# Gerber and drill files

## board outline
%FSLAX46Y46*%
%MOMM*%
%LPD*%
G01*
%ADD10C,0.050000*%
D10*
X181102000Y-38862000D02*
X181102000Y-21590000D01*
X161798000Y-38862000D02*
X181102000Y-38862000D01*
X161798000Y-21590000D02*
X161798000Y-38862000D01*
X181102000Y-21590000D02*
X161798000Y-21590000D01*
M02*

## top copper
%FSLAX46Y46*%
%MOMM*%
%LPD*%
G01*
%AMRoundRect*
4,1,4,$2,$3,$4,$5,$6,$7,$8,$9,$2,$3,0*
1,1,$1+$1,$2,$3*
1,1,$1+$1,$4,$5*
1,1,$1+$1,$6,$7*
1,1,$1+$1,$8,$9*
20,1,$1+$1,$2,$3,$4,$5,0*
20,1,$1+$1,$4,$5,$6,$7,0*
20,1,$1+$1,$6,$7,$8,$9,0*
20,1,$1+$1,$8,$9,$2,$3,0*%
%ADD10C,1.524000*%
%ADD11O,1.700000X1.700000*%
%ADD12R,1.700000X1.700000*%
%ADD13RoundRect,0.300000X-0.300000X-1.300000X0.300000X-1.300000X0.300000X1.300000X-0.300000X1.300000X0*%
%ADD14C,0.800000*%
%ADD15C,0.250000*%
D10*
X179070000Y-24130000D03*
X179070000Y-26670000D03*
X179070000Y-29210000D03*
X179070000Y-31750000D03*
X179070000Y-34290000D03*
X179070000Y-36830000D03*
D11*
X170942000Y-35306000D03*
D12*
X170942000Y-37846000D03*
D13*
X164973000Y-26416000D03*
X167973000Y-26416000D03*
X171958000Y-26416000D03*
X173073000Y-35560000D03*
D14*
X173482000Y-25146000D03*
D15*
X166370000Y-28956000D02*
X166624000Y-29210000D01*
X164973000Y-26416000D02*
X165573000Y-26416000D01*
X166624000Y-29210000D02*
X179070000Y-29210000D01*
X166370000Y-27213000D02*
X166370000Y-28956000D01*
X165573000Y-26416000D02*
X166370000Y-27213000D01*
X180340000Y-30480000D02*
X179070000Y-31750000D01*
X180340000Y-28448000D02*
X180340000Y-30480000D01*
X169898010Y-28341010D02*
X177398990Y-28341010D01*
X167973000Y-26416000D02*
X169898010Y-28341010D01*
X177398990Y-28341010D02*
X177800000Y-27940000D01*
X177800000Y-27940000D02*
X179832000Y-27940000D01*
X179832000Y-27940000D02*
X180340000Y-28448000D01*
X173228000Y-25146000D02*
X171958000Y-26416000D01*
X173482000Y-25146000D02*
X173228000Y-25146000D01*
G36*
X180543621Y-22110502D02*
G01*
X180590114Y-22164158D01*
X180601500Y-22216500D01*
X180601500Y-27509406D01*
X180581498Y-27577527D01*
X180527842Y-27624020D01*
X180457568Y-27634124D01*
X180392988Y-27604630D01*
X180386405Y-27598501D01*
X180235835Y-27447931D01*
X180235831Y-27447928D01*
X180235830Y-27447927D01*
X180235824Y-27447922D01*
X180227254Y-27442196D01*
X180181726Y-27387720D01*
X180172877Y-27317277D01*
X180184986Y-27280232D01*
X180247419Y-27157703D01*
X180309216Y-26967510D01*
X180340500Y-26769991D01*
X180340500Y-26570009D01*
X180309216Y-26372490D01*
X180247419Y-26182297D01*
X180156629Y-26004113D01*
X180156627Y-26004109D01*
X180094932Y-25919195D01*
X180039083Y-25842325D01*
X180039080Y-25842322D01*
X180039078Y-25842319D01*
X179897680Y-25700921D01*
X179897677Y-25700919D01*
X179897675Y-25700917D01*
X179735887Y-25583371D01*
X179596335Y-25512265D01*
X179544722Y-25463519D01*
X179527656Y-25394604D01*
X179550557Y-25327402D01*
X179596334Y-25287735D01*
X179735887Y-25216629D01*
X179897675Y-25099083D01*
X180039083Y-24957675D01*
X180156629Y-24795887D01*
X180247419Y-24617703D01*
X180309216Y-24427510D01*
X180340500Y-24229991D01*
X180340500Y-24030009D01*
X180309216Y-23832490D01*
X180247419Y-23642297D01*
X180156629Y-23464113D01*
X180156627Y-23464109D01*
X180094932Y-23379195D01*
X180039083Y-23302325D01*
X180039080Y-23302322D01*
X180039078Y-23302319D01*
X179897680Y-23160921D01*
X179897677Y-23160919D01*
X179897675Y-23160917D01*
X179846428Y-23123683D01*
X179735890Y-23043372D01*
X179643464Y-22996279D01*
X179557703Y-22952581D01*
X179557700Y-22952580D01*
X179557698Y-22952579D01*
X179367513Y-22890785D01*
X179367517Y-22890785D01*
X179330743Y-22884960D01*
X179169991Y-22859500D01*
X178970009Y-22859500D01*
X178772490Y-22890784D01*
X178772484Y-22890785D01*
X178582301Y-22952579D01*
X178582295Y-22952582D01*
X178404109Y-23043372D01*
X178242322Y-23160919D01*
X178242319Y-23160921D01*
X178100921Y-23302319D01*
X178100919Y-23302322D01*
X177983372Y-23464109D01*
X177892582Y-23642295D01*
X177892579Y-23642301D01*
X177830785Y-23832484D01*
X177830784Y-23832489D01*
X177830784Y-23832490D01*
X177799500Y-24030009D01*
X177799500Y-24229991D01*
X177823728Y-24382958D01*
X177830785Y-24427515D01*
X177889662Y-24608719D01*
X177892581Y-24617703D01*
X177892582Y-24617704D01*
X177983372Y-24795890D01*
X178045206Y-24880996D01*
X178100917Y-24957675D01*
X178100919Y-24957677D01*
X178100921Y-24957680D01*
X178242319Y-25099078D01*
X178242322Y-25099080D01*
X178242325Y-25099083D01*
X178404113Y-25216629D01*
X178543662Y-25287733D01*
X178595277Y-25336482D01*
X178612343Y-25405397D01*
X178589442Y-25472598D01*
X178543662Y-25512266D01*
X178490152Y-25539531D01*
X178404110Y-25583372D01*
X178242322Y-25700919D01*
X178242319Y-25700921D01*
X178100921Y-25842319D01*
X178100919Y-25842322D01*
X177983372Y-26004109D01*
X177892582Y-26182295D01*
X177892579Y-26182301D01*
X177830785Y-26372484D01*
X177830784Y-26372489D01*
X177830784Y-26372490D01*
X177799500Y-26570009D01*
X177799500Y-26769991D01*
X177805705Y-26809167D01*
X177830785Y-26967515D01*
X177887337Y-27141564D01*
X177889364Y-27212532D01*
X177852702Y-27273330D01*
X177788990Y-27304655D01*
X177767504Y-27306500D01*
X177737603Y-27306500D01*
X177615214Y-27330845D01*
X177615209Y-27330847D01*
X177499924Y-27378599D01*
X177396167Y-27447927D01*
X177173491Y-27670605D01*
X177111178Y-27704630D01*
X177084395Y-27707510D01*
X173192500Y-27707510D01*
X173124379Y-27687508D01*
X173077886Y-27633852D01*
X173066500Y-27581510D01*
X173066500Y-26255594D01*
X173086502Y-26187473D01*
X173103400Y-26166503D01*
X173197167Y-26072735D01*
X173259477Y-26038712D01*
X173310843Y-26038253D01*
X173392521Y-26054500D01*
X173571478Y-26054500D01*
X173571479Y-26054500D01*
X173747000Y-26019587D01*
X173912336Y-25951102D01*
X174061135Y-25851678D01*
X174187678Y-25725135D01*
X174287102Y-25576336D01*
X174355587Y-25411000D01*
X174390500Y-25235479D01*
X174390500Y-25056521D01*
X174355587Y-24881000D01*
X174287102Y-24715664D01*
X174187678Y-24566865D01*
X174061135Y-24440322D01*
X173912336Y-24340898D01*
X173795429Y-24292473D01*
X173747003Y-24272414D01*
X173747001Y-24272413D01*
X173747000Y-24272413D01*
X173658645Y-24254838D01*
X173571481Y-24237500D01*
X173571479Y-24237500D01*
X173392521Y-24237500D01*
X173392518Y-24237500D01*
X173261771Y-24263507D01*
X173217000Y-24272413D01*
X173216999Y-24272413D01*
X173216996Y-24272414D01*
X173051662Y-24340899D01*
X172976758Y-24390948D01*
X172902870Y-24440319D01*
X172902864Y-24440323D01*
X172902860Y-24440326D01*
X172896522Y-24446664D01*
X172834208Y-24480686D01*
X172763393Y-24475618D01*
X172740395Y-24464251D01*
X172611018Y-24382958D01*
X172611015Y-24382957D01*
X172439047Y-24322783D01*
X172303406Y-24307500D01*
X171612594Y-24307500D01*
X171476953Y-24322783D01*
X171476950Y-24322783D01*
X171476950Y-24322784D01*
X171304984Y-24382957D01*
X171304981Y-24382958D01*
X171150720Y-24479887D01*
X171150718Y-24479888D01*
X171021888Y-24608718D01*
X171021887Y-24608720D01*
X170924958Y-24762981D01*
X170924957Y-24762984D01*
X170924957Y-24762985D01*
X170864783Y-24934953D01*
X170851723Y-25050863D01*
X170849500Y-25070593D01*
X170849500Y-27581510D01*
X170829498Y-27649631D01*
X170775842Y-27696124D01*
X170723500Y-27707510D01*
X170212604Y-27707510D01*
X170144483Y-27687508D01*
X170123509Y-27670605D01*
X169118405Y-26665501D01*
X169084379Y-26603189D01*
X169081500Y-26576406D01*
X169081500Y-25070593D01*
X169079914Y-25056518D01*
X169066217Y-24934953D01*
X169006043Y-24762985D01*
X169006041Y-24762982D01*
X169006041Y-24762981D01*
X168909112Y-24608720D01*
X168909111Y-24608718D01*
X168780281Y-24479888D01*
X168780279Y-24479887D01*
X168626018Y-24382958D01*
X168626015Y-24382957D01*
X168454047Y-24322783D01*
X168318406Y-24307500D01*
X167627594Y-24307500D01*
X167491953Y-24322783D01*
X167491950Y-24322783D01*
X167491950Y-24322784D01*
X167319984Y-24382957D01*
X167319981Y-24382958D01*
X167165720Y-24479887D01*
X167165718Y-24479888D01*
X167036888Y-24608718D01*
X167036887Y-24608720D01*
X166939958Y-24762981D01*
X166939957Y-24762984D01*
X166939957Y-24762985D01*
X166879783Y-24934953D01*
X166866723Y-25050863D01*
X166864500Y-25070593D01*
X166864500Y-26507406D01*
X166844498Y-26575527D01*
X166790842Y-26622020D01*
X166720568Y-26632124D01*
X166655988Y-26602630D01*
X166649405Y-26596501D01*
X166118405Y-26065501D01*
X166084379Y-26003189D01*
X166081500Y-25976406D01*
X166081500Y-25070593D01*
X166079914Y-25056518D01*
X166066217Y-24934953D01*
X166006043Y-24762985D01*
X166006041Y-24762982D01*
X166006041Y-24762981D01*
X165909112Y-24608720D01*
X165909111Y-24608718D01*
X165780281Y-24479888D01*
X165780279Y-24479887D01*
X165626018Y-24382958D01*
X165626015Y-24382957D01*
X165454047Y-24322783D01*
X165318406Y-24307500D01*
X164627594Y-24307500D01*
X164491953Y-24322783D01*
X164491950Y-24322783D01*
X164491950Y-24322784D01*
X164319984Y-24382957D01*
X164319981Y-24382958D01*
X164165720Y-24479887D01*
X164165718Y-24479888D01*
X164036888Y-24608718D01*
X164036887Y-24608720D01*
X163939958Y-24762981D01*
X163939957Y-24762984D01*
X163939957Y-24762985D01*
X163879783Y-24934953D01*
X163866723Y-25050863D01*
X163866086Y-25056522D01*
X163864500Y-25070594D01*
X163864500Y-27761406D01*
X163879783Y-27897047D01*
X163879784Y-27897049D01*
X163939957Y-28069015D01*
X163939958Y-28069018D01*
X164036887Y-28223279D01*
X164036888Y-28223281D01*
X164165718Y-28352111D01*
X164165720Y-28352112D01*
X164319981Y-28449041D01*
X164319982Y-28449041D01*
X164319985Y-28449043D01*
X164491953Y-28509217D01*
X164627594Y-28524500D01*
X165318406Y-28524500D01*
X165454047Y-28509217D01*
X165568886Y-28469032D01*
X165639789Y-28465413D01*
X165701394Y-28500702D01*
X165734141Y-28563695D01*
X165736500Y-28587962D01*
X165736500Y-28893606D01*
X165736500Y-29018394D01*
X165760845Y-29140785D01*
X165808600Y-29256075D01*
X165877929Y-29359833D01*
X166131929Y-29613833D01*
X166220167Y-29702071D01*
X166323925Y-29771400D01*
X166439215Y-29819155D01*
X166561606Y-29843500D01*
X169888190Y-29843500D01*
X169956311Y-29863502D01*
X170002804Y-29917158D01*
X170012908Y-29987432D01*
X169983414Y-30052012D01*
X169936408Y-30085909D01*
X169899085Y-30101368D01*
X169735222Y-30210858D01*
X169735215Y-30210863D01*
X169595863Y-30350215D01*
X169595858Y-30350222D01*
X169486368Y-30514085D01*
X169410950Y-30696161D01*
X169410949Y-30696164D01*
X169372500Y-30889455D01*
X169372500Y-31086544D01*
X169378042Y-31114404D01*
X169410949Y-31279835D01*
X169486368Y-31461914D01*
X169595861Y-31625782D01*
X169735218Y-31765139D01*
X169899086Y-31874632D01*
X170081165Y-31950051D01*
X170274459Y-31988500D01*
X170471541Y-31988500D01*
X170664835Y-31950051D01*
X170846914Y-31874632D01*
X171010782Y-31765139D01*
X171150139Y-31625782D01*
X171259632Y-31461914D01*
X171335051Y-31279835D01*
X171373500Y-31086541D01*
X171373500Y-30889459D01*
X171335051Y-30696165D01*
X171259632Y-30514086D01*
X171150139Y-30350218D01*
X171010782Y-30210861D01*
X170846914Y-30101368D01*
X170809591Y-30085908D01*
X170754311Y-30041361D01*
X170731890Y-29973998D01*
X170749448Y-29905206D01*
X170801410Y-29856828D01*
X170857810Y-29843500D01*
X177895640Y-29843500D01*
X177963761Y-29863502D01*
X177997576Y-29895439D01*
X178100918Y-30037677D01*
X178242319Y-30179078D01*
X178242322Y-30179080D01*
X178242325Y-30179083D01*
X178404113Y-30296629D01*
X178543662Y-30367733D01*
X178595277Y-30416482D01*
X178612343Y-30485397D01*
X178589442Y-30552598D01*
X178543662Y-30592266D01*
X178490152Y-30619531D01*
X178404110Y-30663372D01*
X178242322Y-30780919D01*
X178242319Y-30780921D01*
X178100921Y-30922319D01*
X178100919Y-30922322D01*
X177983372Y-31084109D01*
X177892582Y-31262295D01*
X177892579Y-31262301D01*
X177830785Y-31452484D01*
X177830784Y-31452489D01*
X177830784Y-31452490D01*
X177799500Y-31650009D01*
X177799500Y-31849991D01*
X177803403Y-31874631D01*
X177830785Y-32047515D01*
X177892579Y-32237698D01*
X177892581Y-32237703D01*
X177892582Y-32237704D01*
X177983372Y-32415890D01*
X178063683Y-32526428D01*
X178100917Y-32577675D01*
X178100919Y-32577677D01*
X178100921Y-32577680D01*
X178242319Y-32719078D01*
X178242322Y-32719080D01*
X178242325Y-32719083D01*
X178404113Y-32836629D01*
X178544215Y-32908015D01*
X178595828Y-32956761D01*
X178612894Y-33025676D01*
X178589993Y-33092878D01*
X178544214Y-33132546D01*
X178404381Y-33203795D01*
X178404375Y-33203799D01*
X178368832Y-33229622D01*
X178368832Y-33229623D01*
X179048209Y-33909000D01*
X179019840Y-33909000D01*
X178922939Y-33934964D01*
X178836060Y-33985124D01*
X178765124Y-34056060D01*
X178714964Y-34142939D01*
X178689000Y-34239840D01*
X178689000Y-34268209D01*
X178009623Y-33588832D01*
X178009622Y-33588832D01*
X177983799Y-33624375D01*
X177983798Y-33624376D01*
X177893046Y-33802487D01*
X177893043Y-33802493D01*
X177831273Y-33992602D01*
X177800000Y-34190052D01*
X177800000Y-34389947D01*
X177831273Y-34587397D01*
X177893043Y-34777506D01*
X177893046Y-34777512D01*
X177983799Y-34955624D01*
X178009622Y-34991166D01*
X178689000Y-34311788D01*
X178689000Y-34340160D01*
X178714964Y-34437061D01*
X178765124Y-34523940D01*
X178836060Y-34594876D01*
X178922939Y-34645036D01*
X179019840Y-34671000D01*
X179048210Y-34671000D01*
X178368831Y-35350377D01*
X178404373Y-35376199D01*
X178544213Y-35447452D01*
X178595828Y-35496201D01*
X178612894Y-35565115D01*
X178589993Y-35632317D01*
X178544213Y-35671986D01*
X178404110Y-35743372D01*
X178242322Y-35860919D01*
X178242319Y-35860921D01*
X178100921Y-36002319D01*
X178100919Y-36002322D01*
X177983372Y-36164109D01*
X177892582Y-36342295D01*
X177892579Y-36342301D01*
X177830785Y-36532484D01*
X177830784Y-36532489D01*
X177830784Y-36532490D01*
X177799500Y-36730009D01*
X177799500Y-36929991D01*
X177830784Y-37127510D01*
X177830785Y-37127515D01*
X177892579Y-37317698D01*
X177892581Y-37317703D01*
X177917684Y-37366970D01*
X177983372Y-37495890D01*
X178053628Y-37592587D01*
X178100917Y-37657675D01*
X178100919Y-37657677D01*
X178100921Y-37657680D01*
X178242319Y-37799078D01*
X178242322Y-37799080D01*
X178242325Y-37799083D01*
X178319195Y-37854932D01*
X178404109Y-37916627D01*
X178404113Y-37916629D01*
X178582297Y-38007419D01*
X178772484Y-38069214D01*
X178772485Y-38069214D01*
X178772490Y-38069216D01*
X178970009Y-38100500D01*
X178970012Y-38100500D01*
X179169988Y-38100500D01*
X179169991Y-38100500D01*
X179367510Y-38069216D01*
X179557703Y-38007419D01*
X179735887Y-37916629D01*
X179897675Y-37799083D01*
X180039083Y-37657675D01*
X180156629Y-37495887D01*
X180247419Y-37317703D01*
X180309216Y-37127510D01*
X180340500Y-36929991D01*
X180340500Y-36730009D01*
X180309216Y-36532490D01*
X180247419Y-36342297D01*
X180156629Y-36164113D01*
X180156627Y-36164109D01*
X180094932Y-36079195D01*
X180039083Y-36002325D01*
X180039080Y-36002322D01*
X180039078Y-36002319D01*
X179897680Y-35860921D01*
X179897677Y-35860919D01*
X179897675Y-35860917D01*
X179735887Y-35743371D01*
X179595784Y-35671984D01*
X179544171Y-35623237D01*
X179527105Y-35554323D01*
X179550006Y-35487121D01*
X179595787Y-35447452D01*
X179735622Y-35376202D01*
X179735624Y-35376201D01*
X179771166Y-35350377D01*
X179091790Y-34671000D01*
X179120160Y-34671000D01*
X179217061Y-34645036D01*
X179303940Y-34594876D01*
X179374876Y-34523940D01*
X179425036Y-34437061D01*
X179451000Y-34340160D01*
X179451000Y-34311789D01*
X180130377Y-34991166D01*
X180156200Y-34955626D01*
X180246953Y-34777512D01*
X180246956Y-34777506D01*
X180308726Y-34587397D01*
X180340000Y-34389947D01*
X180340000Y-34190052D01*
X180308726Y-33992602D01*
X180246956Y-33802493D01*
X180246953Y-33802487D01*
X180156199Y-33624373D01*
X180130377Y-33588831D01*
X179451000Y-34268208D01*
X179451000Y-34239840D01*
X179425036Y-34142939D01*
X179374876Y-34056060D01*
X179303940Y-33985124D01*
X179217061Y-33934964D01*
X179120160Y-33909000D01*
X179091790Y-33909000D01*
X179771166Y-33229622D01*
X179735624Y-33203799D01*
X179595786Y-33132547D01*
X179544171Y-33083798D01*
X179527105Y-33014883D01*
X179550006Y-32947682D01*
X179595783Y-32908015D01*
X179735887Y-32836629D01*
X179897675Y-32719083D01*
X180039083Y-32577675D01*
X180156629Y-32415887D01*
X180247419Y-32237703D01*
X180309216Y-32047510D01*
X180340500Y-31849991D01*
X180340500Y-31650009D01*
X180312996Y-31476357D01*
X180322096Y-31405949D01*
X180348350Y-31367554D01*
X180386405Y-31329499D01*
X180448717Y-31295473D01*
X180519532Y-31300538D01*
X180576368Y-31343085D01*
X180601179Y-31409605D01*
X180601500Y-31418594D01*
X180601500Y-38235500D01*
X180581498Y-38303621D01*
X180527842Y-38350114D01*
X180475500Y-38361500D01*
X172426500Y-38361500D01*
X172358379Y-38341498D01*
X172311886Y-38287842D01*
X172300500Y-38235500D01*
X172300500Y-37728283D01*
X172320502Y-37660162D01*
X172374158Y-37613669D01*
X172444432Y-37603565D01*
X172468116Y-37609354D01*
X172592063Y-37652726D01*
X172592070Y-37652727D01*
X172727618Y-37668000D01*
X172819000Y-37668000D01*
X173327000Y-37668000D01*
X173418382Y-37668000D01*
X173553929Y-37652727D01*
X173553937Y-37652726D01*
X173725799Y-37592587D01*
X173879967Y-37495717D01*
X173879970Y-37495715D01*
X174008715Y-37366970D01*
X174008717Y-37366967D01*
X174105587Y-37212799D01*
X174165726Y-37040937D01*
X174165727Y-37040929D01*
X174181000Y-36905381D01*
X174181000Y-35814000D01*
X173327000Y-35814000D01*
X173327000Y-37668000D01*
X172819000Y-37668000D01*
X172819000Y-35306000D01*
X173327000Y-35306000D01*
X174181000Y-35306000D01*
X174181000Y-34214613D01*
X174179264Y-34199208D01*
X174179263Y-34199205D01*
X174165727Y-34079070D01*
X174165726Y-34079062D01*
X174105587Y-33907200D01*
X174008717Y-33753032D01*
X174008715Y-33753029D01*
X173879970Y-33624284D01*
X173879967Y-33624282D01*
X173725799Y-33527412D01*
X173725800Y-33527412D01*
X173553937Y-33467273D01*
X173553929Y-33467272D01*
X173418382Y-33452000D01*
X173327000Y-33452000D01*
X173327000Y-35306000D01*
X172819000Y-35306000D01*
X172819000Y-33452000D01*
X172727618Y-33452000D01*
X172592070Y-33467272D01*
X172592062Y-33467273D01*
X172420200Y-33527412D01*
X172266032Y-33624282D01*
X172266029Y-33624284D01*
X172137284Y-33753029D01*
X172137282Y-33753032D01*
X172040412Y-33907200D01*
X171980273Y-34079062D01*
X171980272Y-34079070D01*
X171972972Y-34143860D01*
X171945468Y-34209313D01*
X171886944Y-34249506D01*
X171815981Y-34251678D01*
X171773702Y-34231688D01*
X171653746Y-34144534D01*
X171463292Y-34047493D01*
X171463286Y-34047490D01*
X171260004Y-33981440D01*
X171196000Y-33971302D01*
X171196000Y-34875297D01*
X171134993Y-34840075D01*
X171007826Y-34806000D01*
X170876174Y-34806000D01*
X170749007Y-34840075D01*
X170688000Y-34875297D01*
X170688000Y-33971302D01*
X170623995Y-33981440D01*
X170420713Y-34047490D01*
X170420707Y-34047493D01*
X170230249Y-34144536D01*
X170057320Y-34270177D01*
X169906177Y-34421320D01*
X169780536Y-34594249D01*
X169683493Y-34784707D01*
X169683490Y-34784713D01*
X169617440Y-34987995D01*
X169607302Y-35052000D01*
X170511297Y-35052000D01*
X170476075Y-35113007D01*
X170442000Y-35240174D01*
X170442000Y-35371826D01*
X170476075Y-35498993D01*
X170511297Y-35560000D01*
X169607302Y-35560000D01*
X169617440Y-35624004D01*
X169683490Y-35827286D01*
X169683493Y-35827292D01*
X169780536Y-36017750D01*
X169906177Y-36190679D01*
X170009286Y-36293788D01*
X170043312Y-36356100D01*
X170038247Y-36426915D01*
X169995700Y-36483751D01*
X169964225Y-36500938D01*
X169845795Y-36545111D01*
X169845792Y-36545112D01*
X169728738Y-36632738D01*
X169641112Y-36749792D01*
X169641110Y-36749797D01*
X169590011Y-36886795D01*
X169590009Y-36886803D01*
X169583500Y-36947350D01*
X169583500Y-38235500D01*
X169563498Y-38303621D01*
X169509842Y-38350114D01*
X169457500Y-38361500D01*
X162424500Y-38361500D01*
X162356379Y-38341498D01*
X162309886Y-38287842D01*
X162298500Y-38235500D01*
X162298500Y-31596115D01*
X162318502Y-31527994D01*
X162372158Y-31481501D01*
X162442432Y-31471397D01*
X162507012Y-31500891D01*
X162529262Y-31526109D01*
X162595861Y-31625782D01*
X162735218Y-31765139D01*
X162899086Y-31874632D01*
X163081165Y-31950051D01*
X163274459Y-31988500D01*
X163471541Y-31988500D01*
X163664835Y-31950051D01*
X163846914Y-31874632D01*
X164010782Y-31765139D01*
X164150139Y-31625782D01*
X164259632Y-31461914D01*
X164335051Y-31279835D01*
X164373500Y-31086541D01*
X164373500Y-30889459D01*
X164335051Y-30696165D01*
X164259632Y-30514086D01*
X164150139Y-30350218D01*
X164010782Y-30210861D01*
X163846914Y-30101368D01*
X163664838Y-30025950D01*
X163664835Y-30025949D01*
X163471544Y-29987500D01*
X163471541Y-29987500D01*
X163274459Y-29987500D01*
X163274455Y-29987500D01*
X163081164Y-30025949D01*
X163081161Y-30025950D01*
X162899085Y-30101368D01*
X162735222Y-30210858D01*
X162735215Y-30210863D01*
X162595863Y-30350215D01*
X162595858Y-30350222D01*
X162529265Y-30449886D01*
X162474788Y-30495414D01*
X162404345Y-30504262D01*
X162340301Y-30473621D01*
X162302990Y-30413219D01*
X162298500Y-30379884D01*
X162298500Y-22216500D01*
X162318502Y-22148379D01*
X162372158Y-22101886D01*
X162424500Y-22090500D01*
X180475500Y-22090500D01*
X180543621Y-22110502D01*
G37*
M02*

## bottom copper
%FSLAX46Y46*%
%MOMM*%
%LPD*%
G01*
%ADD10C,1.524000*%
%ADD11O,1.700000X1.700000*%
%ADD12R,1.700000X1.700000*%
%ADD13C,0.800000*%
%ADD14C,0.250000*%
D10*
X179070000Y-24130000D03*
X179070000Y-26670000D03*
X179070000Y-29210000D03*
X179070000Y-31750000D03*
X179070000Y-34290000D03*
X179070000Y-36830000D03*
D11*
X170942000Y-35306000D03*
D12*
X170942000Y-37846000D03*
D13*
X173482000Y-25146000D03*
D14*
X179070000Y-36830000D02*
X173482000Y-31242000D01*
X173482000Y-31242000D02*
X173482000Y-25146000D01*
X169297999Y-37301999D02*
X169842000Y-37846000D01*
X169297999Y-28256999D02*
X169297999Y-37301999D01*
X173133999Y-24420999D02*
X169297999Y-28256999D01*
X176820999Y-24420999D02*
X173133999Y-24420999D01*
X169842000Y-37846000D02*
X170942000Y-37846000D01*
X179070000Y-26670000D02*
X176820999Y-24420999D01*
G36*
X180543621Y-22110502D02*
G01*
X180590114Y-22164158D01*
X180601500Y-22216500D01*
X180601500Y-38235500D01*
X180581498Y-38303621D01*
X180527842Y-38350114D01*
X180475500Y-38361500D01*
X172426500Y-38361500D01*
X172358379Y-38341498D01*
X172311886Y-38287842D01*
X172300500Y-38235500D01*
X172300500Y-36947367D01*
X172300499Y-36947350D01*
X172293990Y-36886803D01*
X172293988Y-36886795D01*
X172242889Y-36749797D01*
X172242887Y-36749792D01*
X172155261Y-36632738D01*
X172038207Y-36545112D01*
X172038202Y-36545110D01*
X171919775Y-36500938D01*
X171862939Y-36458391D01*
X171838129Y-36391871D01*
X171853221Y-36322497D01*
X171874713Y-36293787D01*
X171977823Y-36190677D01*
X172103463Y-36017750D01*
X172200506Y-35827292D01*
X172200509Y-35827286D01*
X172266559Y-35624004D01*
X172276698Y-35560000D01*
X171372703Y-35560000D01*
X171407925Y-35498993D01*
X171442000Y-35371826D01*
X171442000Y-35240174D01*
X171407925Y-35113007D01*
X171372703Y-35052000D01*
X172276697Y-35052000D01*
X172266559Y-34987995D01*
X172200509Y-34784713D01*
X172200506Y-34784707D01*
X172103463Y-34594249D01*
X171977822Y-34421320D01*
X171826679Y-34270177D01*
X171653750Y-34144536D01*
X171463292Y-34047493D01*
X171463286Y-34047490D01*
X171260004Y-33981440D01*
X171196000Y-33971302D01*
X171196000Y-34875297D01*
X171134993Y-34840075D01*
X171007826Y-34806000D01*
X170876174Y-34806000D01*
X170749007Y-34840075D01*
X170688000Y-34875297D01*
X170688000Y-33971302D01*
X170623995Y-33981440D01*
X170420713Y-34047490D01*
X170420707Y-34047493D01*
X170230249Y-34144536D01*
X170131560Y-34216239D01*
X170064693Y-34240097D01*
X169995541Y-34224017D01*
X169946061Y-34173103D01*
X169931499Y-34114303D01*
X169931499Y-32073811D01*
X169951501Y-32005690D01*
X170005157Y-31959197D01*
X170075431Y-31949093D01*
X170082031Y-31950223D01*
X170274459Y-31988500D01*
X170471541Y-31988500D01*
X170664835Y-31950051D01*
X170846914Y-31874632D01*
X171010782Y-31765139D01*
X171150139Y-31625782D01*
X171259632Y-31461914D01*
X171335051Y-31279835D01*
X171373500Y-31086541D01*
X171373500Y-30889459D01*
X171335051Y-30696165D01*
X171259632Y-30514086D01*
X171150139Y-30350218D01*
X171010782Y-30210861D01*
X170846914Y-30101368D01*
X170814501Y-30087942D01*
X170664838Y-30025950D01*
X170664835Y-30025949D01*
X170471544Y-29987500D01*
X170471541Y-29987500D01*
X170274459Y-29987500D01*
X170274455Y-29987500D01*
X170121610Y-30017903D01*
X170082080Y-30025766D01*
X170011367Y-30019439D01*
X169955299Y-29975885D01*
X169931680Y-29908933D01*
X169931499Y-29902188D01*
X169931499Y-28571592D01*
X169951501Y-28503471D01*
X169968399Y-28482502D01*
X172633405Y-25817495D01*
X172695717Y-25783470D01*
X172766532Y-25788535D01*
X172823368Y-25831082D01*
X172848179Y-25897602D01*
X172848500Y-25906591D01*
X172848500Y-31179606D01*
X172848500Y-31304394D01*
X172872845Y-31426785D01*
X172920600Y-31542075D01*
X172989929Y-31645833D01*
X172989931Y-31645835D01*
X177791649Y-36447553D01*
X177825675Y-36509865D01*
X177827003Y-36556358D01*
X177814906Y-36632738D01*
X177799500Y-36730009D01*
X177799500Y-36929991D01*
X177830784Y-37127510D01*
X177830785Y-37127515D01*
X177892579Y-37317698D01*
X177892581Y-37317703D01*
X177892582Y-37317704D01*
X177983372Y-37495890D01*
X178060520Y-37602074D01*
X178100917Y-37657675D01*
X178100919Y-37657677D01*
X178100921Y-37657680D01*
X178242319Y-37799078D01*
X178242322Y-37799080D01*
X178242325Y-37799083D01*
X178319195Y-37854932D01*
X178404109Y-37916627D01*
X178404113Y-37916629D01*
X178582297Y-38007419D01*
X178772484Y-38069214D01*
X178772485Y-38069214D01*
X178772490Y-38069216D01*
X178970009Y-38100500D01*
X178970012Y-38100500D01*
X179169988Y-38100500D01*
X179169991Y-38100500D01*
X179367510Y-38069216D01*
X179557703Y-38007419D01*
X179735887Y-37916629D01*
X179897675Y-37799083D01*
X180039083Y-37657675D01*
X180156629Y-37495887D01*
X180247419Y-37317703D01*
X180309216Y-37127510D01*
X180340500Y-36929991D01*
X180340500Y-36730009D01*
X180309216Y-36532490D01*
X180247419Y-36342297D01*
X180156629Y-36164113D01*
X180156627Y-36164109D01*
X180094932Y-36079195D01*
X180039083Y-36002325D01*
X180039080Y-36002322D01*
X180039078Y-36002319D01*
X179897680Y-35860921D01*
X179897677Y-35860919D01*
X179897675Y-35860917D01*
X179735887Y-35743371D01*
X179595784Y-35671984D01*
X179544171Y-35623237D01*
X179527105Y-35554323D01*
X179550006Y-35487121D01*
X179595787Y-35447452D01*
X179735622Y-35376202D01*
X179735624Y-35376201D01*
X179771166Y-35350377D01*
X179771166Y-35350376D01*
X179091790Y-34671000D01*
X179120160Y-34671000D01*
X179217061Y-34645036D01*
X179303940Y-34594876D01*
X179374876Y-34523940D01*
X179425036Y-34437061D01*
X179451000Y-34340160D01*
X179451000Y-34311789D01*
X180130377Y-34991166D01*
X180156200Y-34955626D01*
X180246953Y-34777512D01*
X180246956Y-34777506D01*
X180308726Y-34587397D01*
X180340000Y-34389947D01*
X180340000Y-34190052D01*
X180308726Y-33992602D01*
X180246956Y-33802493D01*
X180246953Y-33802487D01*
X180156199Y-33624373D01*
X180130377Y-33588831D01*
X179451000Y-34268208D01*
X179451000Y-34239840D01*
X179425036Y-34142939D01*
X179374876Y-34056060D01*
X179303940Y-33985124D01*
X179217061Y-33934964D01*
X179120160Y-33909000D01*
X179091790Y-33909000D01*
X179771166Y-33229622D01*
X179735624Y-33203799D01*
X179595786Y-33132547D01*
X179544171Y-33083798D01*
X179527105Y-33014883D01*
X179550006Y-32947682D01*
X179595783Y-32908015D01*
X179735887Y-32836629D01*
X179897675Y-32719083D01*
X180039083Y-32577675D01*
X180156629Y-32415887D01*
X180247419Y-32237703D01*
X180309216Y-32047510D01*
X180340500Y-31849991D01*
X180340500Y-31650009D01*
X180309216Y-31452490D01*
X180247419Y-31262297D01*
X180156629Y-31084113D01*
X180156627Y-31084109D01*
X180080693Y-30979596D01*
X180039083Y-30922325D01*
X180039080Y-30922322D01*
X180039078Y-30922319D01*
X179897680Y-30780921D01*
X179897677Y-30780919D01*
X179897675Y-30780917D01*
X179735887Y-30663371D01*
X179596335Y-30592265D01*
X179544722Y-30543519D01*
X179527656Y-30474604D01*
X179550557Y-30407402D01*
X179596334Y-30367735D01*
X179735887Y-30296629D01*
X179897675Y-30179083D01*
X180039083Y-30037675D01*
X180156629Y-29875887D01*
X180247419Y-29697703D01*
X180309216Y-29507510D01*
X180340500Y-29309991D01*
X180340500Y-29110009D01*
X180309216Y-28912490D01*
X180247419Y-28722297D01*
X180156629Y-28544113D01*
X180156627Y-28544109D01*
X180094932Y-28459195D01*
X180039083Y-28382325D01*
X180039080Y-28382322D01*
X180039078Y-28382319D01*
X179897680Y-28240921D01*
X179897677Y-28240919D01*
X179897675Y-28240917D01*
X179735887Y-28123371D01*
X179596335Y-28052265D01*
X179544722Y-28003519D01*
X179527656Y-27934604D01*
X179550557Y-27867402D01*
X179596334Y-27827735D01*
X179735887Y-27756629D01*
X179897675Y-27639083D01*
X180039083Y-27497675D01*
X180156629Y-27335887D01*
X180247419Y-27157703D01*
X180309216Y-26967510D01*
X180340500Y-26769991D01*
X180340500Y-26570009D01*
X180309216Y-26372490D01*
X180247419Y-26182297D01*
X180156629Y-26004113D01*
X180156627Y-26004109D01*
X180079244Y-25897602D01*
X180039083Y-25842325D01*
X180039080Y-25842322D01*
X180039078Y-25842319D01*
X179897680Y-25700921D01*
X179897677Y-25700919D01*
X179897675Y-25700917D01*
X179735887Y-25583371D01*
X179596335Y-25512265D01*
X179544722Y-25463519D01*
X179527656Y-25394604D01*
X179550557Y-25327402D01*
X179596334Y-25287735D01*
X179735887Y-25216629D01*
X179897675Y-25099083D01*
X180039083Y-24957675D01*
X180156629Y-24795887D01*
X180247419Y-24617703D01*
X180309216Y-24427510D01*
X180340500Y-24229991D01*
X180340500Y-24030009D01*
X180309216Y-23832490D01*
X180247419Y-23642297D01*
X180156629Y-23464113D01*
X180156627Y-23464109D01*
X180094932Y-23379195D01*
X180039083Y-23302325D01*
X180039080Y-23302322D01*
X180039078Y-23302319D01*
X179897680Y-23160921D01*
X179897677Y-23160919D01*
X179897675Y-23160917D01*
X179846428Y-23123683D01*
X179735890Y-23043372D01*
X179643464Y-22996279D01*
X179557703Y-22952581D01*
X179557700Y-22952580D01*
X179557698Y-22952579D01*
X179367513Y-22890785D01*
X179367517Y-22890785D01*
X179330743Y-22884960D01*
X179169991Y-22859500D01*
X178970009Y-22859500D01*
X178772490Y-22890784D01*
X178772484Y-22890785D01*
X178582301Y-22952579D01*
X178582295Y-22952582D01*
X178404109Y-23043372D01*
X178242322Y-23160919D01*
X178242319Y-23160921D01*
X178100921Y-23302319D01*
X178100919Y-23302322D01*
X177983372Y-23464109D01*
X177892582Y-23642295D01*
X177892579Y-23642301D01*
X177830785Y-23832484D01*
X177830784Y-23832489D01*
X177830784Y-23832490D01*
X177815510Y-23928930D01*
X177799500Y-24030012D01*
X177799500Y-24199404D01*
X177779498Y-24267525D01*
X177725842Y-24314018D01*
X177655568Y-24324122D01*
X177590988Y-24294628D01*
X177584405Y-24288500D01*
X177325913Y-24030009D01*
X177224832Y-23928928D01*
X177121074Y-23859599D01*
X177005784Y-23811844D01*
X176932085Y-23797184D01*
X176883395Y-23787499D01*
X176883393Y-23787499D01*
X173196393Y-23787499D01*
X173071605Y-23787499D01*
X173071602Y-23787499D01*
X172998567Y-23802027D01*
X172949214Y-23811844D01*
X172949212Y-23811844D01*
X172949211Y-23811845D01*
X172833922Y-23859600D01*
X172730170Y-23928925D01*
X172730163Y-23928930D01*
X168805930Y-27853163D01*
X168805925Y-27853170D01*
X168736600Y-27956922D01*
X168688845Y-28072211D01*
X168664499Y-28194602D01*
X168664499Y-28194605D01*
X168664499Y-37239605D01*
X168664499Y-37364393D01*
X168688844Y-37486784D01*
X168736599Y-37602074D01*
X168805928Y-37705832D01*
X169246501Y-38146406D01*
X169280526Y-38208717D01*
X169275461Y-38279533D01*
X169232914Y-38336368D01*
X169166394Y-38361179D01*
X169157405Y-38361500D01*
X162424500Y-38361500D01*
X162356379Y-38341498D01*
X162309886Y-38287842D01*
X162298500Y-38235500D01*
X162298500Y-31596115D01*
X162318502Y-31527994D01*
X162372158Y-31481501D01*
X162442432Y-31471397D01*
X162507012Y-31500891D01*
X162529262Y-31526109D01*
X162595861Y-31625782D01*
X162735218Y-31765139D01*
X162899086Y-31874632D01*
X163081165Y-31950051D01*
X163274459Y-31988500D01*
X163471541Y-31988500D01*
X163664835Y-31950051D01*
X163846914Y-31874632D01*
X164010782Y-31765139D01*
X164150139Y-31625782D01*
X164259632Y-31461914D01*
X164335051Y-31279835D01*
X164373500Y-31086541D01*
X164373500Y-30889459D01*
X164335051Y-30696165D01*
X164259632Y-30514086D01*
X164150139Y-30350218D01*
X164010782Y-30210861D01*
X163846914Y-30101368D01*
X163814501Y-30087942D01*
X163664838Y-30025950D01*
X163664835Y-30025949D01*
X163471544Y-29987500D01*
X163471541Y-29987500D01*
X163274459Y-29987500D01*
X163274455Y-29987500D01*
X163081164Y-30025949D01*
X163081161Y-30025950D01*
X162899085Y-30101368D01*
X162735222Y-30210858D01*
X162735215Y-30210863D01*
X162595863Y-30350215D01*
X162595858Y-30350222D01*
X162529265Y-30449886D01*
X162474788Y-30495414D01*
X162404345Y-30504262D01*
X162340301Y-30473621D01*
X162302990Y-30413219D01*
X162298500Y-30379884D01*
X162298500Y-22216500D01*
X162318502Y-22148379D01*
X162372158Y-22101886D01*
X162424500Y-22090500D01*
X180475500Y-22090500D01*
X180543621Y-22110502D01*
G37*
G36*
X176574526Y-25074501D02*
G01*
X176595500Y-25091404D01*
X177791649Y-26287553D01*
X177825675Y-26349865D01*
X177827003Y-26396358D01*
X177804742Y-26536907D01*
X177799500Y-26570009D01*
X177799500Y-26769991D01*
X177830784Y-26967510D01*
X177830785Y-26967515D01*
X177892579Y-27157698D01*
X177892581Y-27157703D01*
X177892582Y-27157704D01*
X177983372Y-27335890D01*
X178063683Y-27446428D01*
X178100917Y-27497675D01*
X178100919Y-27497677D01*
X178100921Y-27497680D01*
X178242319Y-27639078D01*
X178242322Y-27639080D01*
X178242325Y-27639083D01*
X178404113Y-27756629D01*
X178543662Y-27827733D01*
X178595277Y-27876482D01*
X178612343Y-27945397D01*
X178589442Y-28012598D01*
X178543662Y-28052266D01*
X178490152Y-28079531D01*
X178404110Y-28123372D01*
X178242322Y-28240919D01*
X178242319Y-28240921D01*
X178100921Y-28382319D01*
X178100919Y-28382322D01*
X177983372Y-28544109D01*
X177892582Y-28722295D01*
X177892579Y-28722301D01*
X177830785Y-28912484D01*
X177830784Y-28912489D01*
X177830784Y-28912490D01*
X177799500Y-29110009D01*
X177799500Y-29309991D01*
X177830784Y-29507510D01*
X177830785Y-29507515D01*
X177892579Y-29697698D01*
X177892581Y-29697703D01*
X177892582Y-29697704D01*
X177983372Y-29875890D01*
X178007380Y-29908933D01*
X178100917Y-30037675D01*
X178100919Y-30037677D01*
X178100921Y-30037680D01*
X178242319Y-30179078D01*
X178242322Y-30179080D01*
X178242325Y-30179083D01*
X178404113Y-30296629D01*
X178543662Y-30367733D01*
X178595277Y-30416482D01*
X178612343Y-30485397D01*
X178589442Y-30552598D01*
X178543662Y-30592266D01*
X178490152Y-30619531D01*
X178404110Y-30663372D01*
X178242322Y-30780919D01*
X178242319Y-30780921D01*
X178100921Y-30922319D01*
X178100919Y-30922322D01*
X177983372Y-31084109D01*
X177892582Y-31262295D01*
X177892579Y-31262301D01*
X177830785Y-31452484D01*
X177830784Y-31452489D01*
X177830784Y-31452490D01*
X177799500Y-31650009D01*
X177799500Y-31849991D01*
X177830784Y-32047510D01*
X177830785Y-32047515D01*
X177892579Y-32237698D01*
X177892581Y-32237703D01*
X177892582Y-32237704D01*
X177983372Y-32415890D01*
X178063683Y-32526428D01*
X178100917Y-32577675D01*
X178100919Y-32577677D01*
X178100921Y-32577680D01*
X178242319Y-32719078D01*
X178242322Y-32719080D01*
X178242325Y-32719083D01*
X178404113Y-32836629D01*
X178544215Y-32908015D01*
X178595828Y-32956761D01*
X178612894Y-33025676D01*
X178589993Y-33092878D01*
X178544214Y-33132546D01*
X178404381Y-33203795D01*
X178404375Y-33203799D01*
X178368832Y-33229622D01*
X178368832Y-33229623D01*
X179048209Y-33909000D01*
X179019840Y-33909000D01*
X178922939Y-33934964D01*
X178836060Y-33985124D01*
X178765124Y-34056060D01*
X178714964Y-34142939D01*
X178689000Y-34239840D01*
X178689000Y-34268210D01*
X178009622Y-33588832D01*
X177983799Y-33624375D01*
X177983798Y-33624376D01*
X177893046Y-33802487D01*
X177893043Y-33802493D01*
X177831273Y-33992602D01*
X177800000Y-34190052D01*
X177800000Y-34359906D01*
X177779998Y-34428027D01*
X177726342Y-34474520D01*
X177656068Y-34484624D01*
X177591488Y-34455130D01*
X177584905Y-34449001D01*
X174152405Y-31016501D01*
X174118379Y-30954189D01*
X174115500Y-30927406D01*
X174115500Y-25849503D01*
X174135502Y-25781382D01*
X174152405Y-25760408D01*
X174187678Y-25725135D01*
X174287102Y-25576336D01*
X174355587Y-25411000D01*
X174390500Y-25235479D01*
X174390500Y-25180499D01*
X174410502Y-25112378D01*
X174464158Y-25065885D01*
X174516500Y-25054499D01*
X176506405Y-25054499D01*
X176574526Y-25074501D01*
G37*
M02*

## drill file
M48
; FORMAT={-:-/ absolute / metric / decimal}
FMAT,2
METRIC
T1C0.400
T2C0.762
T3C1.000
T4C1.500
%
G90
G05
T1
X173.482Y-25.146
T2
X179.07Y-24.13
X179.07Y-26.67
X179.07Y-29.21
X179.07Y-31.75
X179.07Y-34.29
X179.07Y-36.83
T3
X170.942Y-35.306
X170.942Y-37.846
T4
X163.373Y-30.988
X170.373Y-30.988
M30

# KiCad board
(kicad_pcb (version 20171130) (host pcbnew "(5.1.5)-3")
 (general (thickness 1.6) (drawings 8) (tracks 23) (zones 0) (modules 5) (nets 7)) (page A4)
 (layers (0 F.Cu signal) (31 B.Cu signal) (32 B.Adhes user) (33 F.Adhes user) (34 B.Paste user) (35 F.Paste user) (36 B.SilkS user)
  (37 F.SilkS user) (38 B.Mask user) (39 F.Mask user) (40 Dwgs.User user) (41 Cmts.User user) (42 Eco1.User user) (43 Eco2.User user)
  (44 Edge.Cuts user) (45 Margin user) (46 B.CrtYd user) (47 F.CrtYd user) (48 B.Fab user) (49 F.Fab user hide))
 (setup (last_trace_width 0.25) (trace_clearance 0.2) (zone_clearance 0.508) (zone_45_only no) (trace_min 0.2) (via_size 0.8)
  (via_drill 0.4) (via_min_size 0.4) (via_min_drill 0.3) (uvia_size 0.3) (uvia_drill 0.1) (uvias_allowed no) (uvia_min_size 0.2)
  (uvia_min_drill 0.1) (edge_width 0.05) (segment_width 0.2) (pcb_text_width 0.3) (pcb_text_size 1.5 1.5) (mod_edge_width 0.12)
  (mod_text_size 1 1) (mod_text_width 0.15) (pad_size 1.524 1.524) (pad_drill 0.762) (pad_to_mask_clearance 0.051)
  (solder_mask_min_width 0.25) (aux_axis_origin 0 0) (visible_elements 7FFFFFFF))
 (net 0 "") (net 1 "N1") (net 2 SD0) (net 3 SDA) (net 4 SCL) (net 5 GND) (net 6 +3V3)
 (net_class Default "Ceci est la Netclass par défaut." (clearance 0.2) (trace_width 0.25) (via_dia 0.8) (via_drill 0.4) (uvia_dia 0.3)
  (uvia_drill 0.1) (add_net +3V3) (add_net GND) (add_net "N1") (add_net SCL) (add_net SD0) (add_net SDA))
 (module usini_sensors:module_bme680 (layer F.Cu) (at 179.07 24.13 180)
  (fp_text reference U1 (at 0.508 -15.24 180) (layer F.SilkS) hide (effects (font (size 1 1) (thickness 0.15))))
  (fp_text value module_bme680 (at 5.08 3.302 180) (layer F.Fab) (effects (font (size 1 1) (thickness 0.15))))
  (pad 6 thru_hole circle (at 0 0 180) (size 1.524 1.524) (drill 0.762) (layers *.Cu *.Mask) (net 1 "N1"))
  (pad 5 thru_hole circle (at 0 -2.54 180) (size 1.524 1.524) (drill 0.762) (layers *.Cu *.Mask) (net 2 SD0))
  (pad 4 thru_hole circle (at 0 -5.08 180) (size 1.524 1.524) (drill 0.762) (layers *.Cu *.Mask) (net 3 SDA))
  (pad 3 thru_hole circle (at 0 -7.62 180) (size 1.524 1.524) (drill 0.762) (layers *.Cu *.Mask) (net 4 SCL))
  (pad 2 thru_hole circle (at 0 -10.16 180) (size 1.524 1.524) (drill 0.762) (layers *.Cu *.Mask) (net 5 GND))
  (pad 1 thru_hole circle (at 0 -12.7 180) (size 1.524 1.524) (drill 0.762) (layers *.Cu *.Mask) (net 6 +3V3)))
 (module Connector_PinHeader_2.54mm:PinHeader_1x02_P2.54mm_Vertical (layer F.Cu) (at 170.942 37.846 180)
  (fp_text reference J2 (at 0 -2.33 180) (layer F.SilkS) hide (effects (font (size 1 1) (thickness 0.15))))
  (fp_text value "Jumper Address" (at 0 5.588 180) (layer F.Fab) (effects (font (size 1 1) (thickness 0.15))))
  (pad 2 thru_hole oval (at 0 2.54 180) (size 1.7 1.7) (drill 1) (layers *.Cu *.Mask) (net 5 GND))
  (pad 1 thru_hole rect (at 0 0 180) (size 1.7 1.7) (drill 1) (layers *.Cu *.Mask) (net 2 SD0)))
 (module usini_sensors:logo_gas (layer B.Cu) (at 165.608 26.416 180)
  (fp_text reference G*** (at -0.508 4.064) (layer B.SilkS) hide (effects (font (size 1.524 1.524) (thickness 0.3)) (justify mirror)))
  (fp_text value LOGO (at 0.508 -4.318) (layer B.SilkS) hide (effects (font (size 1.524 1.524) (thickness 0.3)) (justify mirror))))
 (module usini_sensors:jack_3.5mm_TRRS (layer F.Cu) (at 168.148 30.988)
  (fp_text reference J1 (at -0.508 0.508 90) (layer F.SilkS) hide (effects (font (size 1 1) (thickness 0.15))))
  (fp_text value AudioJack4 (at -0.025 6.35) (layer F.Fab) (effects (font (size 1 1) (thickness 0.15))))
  (pad "" np_thru_hole circle (at 2.225 0) (size 1.5 1.5) (drill 1.5) (layers *.Cu *.Mask))
  (pad "" np_thru_hole circle (at -4.775 0) (size 1.5 1.5) (drill 1.5) (layers *.Cu *.Mask))
  (pad R2 smd roundrect (at -3.175 -4.572) (size 1.2 3.2) (layers F.Cu F.Paste F.Mask) (roundrect_rratio 0.25) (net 3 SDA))
  (pad R1 smd roundrect (at -0.175 -4.572) (size 1.2 3.2) (layers F.Cu F.Paste F.Mask) (roundrect_rratio 0.25) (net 4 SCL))
  (pad T smd roundrect (at 3.81 -4.572) (size 1.2 3.2) (layers F.Cu F.Paste F.Mask) (roundrect_rratio 0.25) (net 6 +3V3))
  (pad S smd roundrect (at 4.925 4.572) (size 1.2 3.2) (layers F.Cu F.Paste F.Mask) (roundrect_rratio 0.25) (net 5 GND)))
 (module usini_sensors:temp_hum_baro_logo (layer B.Cu) (at 172.974 26.416 180)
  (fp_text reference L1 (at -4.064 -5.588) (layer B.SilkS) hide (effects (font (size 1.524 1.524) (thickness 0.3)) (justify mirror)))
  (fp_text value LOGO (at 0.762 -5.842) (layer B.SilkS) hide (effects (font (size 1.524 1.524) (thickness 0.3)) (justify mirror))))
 (gr_line (start 181.102 38.862) (end 181.102 21.59) (layer Edge.Cuts) (width 0.05))
 (gr_line (start 161.798 38.862) (end 181.102 38.862) (layer Edge.Cuts) (width 0.05))
 (gr_line (start 161.798 21.59) (end 161.798 38.862) (layer Edge.Cuts) (width 0.05))
 (gr_line (start 181.102 21.59) (end 161.798 21.59) (layer Edge.Cuts) (width 0.05))
 (segment (start 166.37 28.956) (end 166.624 29.21) (width 0.25) (layer F.Cu) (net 3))
 (segment (start 164.973 26.416) (end 165.573 26.416) (width 0.25) (layer F.Cu) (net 3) (status 10))
 (segment (start 166.624 29.21) (end 179.07 29.21) (width 0.25) (layer F.Cu) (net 3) (status 20))
 (segment (start 166.37 27.213) (end 166.37 28.956) (width 0.25) (layer F.Cu) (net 3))
 (segment (start 165.573 26.416) (end 166.37 27.213) (width 0.25) (layer F.Cu) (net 3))
 (segment (start 180.34 30.48) (end 179.07 31.75) (width 0.25) (layer F.Cu) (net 4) (status 20))
 (segment (start 180.34 28.448) (end 180.34 30.48) (width 0.25) (layer F.Cu) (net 4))
 (segment (start 169.89801 28.34101) (end 177.39899 28.34101) (width 0.25) (layer F.Cu) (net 4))
 (segment (start 167.973 26.416) (end 169.89801 28.34101) (width 0.25) (layer F.Cu) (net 4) (status 10))
 (segment (start 177.39899 28.34101) (end 177.8 27.94) (width 0.25) (layer F.Cu) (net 4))
 (segment (start 177.8 27.94) (end 179.832 27.94) (width 0.25) (layer F.Cu) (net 4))
 (segment (start 179.832 27.94) (end 180.34 28.448) (width 0.25) (layer F.Cu) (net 4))
 (via (at 173.482 25.146) (size 0.8) (drill 0.4) (layers F.Cu B.Cu) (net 6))
 (segment (start 179.07 36.83) (end 173.482 31.242) (width 0.25) (layer B.Cu) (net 6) (status 10))
 (segment (start 173.482 31.242) (end 173.482 25.146) (width 0.25) (layer B.Cu) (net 6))
 (segment (start 173.228 25.146) (end 171.958 26.416) (width 0.25) (layer F.Cu) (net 6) (status 20))
 (segment (start 173.482 25.146) (end 173.228 25.146) (width 0.25) (layer F.Cu) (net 6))
 (segment (start 169.297999 37.301999) (end 169.842 37.846) (width 0.25) (layer B.Cu) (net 2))
 (segment (start 169.297999 28.256999) (end 169.297999 37.301999) (width 0.25) (layer B.Cu) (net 2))
 (segment (start 173.133999 24.420999) (end 169.297999 28.256999) (width 0.25) (layer B.Cu) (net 2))
 (segment (start 176.820999 24.420999) (end 173.133999 24.420999) (width 0.25) (layer B.Cu) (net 2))
 (segment (start 169.842 37.846) (end 170.942 37.846) (width 0.25) (layer B.Cu) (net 2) (status 20))
 (segment (start 179.07 26.67) (end 176.820999 24.420999) (width 0.25) (layer B.Cu) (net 2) (status 10))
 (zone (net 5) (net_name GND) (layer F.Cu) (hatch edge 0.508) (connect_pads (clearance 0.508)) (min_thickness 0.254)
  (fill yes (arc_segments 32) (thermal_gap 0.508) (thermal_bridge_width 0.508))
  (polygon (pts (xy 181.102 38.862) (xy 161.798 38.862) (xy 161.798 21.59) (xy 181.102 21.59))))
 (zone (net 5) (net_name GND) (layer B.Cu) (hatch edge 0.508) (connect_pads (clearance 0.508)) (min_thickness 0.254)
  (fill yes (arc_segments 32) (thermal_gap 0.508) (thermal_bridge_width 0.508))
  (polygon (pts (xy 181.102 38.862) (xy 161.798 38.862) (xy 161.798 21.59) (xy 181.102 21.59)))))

